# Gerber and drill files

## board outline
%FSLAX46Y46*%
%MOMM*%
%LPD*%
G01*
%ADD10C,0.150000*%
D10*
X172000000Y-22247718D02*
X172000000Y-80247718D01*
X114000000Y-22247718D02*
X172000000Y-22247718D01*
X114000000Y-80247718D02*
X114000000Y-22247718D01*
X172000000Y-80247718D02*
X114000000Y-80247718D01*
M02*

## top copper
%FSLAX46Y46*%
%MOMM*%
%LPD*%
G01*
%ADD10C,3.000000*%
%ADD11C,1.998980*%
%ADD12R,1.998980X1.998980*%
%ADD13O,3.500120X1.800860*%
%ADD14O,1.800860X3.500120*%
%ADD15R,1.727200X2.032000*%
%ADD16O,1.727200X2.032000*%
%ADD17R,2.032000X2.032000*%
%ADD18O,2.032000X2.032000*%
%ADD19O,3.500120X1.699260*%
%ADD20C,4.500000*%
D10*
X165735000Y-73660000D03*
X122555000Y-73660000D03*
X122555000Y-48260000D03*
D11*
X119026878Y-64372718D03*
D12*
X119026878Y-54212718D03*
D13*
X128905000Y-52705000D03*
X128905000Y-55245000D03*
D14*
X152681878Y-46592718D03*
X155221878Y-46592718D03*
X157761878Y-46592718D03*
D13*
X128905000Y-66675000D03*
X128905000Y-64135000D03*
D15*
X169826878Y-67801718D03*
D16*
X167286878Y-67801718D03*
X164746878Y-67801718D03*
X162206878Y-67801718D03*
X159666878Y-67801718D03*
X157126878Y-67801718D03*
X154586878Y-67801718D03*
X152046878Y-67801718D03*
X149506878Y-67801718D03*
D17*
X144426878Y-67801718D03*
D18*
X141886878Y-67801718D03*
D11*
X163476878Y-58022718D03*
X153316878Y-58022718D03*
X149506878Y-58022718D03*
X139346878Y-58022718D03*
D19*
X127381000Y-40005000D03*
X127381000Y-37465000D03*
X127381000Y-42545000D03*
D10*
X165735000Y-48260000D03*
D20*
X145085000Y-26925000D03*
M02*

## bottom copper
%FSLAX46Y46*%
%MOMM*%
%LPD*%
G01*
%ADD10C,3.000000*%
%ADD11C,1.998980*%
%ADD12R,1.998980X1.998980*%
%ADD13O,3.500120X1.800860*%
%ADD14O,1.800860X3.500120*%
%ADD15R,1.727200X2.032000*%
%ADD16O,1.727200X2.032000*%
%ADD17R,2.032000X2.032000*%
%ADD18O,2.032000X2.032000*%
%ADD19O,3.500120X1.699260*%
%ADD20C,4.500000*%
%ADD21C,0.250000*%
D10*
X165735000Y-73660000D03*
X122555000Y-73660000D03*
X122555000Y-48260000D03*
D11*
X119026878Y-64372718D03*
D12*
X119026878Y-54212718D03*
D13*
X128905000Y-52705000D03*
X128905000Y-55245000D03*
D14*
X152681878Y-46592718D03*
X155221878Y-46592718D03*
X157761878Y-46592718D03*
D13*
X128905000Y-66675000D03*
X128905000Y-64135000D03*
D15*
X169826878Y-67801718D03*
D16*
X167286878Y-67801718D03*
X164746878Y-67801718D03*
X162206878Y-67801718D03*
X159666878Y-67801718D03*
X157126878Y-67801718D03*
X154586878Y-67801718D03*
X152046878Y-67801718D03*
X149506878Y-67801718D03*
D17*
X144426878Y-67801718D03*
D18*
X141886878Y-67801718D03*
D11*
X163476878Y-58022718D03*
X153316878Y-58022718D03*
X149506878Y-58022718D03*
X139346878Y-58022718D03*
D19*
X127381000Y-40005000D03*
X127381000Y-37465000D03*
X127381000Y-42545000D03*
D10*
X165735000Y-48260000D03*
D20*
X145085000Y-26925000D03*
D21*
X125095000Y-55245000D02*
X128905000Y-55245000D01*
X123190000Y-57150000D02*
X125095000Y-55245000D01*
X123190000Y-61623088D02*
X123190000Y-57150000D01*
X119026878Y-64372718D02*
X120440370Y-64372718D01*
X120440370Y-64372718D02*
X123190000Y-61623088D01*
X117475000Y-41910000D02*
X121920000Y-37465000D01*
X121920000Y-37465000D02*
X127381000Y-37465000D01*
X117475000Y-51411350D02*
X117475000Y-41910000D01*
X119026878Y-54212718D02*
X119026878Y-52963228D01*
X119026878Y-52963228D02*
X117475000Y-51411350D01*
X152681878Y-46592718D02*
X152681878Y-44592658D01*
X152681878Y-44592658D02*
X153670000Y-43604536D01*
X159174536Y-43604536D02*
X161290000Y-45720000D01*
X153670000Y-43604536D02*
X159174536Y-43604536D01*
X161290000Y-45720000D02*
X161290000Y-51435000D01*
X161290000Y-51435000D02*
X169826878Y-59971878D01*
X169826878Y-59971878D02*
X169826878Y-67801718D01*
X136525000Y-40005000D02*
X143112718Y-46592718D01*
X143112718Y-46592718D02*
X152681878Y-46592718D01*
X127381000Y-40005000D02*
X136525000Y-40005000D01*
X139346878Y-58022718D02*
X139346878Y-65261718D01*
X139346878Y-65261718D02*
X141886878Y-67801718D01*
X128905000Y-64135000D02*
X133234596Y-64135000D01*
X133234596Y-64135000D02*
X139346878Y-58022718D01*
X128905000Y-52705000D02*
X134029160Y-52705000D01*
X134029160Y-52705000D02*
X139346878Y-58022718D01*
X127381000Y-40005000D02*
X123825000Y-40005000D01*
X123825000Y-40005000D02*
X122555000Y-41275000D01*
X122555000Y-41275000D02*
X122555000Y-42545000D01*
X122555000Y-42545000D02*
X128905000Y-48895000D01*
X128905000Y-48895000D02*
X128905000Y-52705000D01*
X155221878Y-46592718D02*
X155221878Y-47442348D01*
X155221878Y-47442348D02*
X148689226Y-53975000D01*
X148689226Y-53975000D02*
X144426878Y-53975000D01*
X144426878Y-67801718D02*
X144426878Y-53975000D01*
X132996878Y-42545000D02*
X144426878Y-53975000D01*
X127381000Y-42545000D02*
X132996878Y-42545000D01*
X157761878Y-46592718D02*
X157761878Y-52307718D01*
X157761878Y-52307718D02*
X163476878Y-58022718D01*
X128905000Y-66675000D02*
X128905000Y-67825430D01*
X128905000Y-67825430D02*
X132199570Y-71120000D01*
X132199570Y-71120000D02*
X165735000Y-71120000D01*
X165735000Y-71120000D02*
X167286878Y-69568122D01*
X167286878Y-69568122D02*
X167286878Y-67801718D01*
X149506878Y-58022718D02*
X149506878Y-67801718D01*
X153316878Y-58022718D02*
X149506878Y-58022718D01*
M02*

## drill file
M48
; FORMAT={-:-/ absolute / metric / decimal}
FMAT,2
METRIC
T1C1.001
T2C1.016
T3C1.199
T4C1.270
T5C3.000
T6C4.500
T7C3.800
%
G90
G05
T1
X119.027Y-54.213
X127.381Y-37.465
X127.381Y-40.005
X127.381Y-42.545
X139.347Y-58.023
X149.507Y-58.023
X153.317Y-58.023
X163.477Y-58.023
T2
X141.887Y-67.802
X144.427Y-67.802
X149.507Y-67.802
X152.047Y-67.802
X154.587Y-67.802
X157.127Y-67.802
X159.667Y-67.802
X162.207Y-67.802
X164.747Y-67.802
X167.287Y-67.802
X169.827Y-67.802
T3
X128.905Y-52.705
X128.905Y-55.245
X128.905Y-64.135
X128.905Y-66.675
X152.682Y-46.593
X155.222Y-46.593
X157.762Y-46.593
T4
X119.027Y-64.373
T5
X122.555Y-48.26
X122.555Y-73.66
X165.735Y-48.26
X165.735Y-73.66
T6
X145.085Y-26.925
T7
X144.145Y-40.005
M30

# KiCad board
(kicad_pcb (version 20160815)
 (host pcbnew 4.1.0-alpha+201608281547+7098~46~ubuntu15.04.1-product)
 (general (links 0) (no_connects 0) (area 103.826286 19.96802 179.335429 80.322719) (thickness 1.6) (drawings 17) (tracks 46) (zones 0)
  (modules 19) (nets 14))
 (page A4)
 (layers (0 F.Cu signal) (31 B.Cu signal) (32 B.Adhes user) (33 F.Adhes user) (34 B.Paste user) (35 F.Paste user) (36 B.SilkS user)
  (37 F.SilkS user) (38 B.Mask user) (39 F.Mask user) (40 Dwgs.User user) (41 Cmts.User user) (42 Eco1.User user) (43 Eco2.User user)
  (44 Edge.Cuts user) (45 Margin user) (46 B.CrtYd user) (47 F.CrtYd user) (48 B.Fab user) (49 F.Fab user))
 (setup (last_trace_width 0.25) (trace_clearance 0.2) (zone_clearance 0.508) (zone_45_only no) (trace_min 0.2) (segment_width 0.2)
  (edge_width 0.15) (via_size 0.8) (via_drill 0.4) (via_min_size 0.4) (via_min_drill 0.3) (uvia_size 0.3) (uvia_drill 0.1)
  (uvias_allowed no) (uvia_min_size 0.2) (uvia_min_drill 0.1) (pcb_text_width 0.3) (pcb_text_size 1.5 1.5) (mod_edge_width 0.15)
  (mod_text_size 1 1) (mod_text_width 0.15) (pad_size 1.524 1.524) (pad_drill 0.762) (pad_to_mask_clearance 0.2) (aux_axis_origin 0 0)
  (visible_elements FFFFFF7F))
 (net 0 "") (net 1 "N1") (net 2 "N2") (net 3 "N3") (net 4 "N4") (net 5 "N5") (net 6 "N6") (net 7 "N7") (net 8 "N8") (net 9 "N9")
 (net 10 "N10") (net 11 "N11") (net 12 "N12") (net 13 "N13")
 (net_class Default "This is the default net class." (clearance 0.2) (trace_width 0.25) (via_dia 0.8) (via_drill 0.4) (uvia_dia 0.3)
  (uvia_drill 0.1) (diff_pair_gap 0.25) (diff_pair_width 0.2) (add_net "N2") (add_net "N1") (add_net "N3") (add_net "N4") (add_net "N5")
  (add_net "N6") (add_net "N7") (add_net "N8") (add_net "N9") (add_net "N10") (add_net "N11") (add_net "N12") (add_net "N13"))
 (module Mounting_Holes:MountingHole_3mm (layer F.Cu) (at 165.735 73.66)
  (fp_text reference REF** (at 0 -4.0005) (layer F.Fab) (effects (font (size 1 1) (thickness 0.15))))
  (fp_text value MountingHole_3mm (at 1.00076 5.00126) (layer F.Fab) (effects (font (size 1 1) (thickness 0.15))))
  (pad 1 thru_hole circle (at 0 0) (size 3 3) (drill 3) (layers)))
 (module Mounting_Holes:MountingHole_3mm (layer F.Cu) (at 122.555 73.66)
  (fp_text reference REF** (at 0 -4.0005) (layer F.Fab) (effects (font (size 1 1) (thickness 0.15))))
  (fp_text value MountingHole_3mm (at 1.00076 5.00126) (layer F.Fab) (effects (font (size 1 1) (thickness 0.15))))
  (pad 1 thru_hole circle (at 0 0) (size 3 3) (drill 3) (layers)))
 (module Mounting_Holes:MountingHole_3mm (layer F.Cu) (at 122.555 48.26)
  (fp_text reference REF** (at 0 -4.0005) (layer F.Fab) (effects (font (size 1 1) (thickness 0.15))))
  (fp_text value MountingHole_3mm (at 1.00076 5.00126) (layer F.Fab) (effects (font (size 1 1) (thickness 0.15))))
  (pad 1 thru_hole circle (at 0 0) (size 3 3) (drill 3) (layers)))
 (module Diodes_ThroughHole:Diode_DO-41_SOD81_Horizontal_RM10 (layer F.Cu) (at 119.024338 54.212718 270)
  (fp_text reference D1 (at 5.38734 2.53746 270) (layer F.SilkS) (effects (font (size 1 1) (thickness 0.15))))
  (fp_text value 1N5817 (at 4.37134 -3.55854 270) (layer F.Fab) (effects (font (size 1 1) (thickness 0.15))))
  (pad 2 thru_hole circle (at 10.16 -0.00254 90) (size 1.99898 1.99898) (drill 1.27) (layers *.Cu *.Mask F.SilkS) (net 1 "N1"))
  (pad 1 thru_hole rect (at 0 -0.00254 90) (size 1.99898 1.99898) (drill 1.00076) (layers *.Cu *.Mask F.SilkS) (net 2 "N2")))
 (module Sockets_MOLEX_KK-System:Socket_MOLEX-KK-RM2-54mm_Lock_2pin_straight (layer F.Cu) (at 128.905 53.975 270)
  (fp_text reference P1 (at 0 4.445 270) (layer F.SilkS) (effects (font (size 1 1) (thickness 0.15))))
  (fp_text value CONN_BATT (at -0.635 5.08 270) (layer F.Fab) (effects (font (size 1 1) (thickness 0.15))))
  (pad 1 thru_hole oval (at -1.27 0 270) (size 1.80086 3.50012) (drill 1.19888) (layers *.Cu *.Mask F.SilkS) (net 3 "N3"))
  (pad 2 thru_hole oval (at 1.27 0 270) (size 1.80086 3.50012) (drill 1.19888) (layers *.Cu *.Mask F.SilkS) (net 1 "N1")))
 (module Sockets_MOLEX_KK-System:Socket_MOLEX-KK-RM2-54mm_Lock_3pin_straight (layer F.Cu) (at 155.221878 46.592718)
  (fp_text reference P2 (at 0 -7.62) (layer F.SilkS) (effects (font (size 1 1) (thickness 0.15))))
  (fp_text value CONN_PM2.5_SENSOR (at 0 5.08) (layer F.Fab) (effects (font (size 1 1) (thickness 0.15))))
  (pad 1 thru_hole oval (at -2.54 0) (size 1.80086 3.50012) (drill 1.19888) (layers *.Cu *.Mask F.SilkS) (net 3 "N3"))
  (pad 2 thru_hole oval (at 0 0) (size 1.80086 3.50012) (drill 1.19888) (layers *.Cu *.Mask F.SilkS) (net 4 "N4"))
  (pad 3 thru_hole oval (at 2.54 0) (size 1.80086 3.50012) (drill 1.19888) (layers *.Cu *.Mask F.SilkS) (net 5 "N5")))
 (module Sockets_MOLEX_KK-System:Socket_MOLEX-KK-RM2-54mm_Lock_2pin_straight (layer F.Cu) (at 128.905 65.405 90)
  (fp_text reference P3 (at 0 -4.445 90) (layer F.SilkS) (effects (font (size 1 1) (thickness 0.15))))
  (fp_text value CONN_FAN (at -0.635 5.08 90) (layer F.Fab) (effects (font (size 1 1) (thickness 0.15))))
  (pad 1 thru_hole oval (at -1.27 0 90) (size 1.80086 3.50012) (drill 1.19888) (layers *.Cu *.Mask F.SilkS) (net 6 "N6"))
  (pad 2 thru_hole oval (at 1.27 0 90) (size 1.80086 3.50012) (drill 1.19888) (layers *.Cu *.Mask F.SilkS) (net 3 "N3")))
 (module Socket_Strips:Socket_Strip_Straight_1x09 (layer F.Cu) (at 169.826878 67.801718 180)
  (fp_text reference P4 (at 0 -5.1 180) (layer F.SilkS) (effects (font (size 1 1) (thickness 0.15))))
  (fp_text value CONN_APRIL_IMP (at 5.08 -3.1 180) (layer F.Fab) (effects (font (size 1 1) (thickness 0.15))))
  (pad 1 thru_hole rect (at 0 0 180) (size 1.7272 2.032) (drill 1.016) (layers *.Cu *.Mask F.SilkS) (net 3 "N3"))
  (pad 2 thru_hole oval (at 2.54 0 180) (size 1.7272 2.032) (drill 1.016) (layers *.Cu *.Mask F.SilkS) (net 6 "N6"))
  (pad 3 thru_hole oval (at 5.08 0 180) (size 1.7272 2.032) (drill 1.016) (layers *.Cu *.Mask F.SilkS) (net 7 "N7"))
  (pad 4 thru_hole oval (at 7.62 0 180) (size 1.7272 2.032) (drill 1.016) (layers *.Cu *.Mask F.SilkS) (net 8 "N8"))
  (pad 5 thru_hole oval (at 10.16 0 180) (size 1.7272 2.032) (drill 1.016) (layers *.Cu *.Mask F.SilkS) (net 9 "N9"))
  (pad 6 thru_hole oval (at 12.7 0 180) (size 1.7272 2.032) (drill 1.016) (layers *.Cu *.Mask F.SilkS) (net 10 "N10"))
  (pad 7 thru_hole oval (at 15.24 0 180) (size 1.7272 2.032) (drill 1.016) (layers *.Cu *.Mask F.SilkS) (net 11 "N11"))
  (pad 8 thru_hole oval (at 17.78 0 180) (size 1.7272 2.032) (drill 1.016) (layers *.Cu *.Mask F.SilkS) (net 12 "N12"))
  (pad 9 thru_hole oval (at 20.32 0 180) (size 1.7272 2.032) (drill 1.016) (layers *.Cu *.Mask F.SilkS) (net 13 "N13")))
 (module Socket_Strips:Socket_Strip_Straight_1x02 (layer F.Cu) (at 144.426878 67.801718 180)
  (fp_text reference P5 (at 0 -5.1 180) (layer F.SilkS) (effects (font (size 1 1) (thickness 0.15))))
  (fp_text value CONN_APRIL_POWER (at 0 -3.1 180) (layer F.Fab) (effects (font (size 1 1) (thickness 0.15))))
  (pad 1 thru_hole rect (at 0 0 180) (size 2.032 2.032) (drill 1.016) (layers *.Cu *.Mask F.SilkS) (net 4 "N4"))
  (pad 2 thru_hole oval (at 2.54 0 180) (size 2.032 2.032) (drill 1.016) (layers *.Cu *.Mask F.SilkS) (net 3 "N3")))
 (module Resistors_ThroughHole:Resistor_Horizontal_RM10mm (layer F.Cu) (at 158.396878 58.022718 180)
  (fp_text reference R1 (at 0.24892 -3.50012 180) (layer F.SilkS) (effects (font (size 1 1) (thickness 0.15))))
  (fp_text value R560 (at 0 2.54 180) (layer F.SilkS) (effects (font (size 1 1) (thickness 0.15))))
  (pad 1 thru_hole circle (at -5.08 0 180) (size 1.99898 1.99898) (drill 1.00076) (layers *.Cu *.SilkS *.Mask) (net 5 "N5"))
  (pad 2 thru_hole circle (at 5.08 0 180) (size 1.99898 1.99898) (drill 1.00076) (layers *.Cu *.SilkS *.Mask) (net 13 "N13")))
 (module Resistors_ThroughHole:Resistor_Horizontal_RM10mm (layer F.Cu) (at 144.426878 58.022718 180)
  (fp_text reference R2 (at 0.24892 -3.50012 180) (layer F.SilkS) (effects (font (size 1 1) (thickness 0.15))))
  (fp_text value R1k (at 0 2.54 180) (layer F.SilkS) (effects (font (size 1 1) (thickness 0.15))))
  (pad 1 thru_hole circle (at -5.08 0 180) (size 1.99898 1.99898) (drill 1.00076) (layers *.Cu *.SilkS *.Mask) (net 13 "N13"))
  (pad 2 thru_hole circle (at 5.08 0 180) (size 1.99898 1.99898) (drill 1.00076) (layers *.Cu *.SilkS *.Mask) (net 3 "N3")))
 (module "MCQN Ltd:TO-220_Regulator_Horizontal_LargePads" (layer F.Cu) (at 127.381 40.005 270)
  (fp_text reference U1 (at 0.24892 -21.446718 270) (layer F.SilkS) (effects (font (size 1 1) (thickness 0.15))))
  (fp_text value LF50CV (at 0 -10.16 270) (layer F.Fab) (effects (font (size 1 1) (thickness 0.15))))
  (pad GND thru_hole oval (at 0 0) (size 3.50012 1.69926) (drill 1.00076) (layers *.Cu *.Mask F.SilkS) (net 3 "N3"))
  (pad VI thru_hole oval (at -2.54 0) (size 3.50012 1.69926) (drill 1.00076) (layers *.Cu *.Mask F.SilkS) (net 2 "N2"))
  (pad VO thru_hole oval (at 2.54 0) (size 3.50012 1.69926) (drill 1.00076) (layers *.Cu *.Mask F.SilkS) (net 4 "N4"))
  (pad "" np_thru_hole circle (at 0 -16.764) (size 3.79984 3.79984) (drill 3.79984) (layers *.Cu *.Mask F.SilkS)))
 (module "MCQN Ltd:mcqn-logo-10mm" (layer F.Cu) (at 165.487038 27.760574)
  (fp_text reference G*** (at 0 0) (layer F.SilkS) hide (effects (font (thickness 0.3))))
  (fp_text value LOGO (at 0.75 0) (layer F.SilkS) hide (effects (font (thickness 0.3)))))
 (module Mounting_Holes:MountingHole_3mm (layer F.Cu) (at 165.735 48.26)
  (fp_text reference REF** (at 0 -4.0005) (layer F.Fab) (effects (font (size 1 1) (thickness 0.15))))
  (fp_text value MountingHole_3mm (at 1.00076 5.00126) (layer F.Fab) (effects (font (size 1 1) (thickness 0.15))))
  (pad 1 thru_hole circle (at 0 0) (size 3 3) (drill 3) (layers)))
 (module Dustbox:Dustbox (layer F.Cu) (at 175.26 35.56)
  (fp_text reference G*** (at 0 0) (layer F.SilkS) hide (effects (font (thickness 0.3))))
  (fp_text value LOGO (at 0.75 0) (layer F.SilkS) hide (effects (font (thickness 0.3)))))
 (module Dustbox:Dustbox (layer F.Cu) (at 106.68 29.21)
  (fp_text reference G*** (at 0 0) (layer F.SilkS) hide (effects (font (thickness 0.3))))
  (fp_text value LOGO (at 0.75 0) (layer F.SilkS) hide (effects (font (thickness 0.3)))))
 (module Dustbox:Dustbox (layer F.Cu) (at 126.365 26.035)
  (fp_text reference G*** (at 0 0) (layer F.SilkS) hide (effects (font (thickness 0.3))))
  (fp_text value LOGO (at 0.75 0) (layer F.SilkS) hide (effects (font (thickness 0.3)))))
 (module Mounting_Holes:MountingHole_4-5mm (layer F.Cu) (at 145.085 26.925)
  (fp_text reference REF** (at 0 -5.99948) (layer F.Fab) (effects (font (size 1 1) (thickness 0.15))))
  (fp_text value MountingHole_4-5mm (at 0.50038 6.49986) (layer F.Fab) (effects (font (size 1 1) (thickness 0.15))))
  (pad 1 thru_hole circle (at 0 0) (size 4.5 4.5) (drill 4.5) (layers)))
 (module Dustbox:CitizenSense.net (layer F.Cu) (at 126.238 29.718)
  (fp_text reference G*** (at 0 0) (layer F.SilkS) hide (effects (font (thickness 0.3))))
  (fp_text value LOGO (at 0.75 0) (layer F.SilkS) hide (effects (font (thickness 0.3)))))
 (gr_line (start 172 22.247718) (end 172 80.247718) (layer Edge.Cuts) (width 0.15))
 (gr_line (start 114 22.247718) (end 172 22.247718) (layer Edge.Cuts) (width 0.15))
 (gr_line (start 114 80.247718) (end 114 22.247718) (layer Edge.Cuts) (width 0.15))
 (gr_line (start 172 80.247718) (end 114 80.247718) (layer Edge.Cuts) (width 0.15))
 (segment (start 125.095 55.245) (end 128.905 55.245) (width 0.25) (layer B.Cu) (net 1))
 (segment (start 123.19 57.15) (end 125.095 55.245) (width 0.25) (layer B.Cu) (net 1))
 (segment (start 123.19 61.623088) (end 123.19 57.15) (width 0.25) (layer B.Cu) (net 1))
 (segment (start 119.026878 64.372718) (end 120.44037 64.372718) (width 0.25) (layer B.Cu) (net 1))
 (segment (start 120.44037 64.372718) (end 123.19 61.623088) (width 0.25) (layer B.Cu) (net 1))
 (segment (start 117.475 41.91) (end 121.92 37.465) (width 0.25) (layer B.Cu) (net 2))
 (segment (start 121.92 37.465) (end 127.381 37.465) (width 0.25) (layer B.Cu) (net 2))
 (segment (start 117.475 51.41135) (end 117.475 41.91) (width 0.25) (layer B.Cu) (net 2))
 (segment (start 119.026878 54.212718) (end 119.026878 52.963228) (width 0.25) (layer B.Cu) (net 2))
 (segment (start 119.026878 52.963228) (end 117.475 51.41135) (width 0.25) (layer B.Cu) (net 2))
 (segment (start 152.681878 46.592718) (end 152.681878 44.592658) (width 0.25) (layer B.Cu) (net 3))
 (segment (start 152.681878 44.592658) (end 153.67 43.604536) (width 0.25) (layer B.Cu) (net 3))
 (segment (start 159.174536 43.604536) (end 161.29 45.72) (width 0.25) (layer B.Cu) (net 3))
 (segment (start 153.67 43.604536) (end 159.174536 43.604536) (width 0.25) (layer B.Cu) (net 3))
 (segment (start 161.29 45.72) (end 161.29 51.435) (width 0.25) (layer B.Cu) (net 3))
 (segment (start 161.29 51.435) (end 169.826878 59.971878) (width 0.25) (layer B.Cu) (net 3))
 (segment (start 169.826878 59.971878) (end 169.826878 67.801718) (width 0.25) (layer B.Cu) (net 3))
 (segment (start 136.525 40.005) (end 143.112718 46.592718) (width 0.25) (layer B.Cu) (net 3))
 (segment (start 143.112718 46.592718) (end 152.681878 46.592718) (width 0.25) (layer B.Cu) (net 3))
 (segment (start 127.381 40.005) (end 136.525 40.005) (width 0.25) (layer B.Cu) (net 3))
 (segment (start 139.346878 58.022718) (end 139.346878 65.261718) (width 0.25) (layer B.Cu) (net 3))
 (segment (start 139.346878 65.261718) (end 141.886878 67.801718) (width 0.25) (layer B.Cu) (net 3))
 (segment (start 128.905 64.135) (end 133.234596 64.135) (width 0.25) (layer B.Cu) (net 3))
 (segment (start 133.234596 64.135) (end 139.346878 58.022718) (width 0.25) (layer B.Cu) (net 3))
 (segment (start 128.905 52.705) (end 134.02916 52.705) (width 0.25) (layer B.Cu) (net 3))
 (segment (start 134.02916 52.705) (end 139.346878 58.022718) (width 0.25) (layer B.Cu) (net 3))
 (segment (start 127.381 40.005) (end 123.825 40.005) (width 0.25) (layer B.Cu) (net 3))
 (segment (start 123.825 40.005) (end 122.555 41.275) (width 0.25) (layer B.Cu) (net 3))
 (segment (start 122.555 41.275) (end 122.555 42.545) (width 0.25) (layer B.Cu) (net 3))
 (segment (start 122.555 42.545) (end 128.905 48.895) (width 0.25) (layer B.Cu) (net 3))
 (segment (start 128.905 48.895) (end 128.905 52.705) (width 0.25) (layer B.Cu) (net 3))
 (segment (start 155.221878 46.592718) (end 155.221878 47.442348) (width 0.25) (layer B.Cu) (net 4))
 (segment (start 155.221878 47.442348) (end 148.689226 53.975) (width 0.25) (layer B.Cu) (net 4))
 (segment (start 148.689226 53.975) (end 144.426878 53.975) (width 0.25) (layer B.Cu) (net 4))
 (segment (start 144.426878 67.801718) (end 144.426878 53.975) (width 0.25) (layer B.Cu) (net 4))
 (segment (start 132.996878 42.545) (end 144.426878 53.975) (width 0.25) (layer B.Cu) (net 4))
 (segment (start 127.381 42.545) (end 132.996878 42.545) (width 0.25) (layer B.Cu) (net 4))
 (segment (start 157.761878 46.592718) (end 157.761878 52.307718) (width 0.25) (layer B.Cu) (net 5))
 (segment (start 157.761878 52.307718) (end 163.476878 58.022718) (width 0.25) (layer B.Cu) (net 5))
 (segment (start 128.905 66.675) (end 128.905 67.82543) (width 0.25) (layer B.Cu) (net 6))
 (segment (start 128.905 67.82543) (end 132.19957 71.12) (width 0.25) (layer B.Cu) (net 6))
 (segment (start 132.19957 71.12) (end 165.735 71.12) (width 0.25) (layer B.Cu) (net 6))
 (segment (start 165.735 71.12) (end 167.286878 69.568122) (width 0.25) (layer B.Cu) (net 6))
 (segment (start 167.286878 69.568122) (end 167.286878 67.801718) (width 0.25) (layer B.Cu) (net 6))
 (segment (start 149.506878 58.022718) (end 149.506878 67.801718) (width 0.25) (layer B.Cu) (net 13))
 (segment (start 153.316878 58.022718) (end 149.506878 58.022718) (width 0.25) (layer B.Cu) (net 13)))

